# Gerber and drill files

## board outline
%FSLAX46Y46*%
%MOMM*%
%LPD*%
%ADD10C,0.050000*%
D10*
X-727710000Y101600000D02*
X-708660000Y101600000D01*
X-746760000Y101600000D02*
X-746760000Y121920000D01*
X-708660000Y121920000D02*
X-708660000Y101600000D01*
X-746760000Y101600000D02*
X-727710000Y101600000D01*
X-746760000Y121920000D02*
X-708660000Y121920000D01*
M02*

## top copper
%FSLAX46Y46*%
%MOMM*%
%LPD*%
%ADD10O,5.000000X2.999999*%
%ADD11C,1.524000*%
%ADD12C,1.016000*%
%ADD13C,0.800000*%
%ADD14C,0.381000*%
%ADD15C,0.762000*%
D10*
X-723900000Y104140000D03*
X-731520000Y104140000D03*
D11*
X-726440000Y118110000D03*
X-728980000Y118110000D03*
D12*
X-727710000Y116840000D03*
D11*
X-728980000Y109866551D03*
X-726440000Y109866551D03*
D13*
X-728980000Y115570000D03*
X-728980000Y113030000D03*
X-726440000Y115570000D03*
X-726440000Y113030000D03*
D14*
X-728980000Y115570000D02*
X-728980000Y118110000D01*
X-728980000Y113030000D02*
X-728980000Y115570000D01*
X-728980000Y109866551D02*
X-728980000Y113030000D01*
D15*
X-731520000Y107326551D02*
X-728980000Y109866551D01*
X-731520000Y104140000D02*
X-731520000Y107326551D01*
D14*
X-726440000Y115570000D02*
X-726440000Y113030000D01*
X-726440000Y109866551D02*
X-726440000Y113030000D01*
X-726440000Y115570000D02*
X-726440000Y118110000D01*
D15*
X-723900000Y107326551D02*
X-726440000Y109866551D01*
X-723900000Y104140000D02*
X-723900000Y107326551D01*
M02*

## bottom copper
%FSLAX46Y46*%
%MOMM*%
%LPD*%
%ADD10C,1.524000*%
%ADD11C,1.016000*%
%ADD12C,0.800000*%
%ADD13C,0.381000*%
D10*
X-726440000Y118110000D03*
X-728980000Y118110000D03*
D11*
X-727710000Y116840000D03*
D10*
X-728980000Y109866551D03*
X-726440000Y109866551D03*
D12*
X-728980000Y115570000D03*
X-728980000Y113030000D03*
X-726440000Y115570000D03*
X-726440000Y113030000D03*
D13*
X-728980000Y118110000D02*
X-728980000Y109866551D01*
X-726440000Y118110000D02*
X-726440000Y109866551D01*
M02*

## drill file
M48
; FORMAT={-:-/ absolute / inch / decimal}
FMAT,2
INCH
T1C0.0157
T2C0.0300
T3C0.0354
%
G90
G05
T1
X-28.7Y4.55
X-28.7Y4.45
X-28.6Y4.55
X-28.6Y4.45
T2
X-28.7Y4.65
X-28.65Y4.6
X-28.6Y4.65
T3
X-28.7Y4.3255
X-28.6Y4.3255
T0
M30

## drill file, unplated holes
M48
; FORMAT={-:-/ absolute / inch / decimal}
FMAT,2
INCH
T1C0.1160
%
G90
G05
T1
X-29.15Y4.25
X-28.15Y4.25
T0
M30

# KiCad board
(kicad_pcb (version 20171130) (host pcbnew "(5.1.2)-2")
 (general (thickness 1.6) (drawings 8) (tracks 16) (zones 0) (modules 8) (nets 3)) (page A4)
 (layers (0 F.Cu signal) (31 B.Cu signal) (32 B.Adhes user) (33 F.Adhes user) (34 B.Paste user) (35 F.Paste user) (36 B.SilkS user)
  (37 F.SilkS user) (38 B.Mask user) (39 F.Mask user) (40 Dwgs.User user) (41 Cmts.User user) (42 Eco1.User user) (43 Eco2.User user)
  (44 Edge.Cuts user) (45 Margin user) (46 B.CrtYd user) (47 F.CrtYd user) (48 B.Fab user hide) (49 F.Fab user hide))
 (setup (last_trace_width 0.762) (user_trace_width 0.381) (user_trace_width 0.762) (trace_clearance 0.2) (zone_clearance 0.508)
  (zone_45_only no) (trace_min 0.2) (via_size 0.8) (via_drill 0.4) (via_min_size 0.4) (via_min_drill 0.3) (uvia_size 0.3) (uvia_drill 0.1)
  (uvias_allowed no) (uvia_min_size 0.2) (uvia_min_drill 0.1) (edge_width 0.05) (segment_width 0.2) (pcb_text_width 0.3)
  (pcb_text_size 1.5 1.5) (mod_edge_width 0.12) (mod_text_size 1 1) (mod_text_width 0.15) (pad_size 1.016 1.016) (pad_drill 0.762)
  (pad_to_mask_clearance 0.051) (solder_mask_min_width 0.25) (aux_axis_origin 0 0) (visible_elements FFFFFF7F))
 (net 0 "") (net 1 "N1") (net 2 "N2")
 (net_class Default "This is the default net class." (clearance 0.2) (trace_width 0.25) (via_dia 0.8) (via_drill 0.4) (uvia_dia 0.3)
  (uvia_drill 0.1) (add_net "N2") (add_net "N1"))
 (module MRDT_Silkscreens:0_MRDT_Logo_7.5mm (layer F.Cu) (at -714.375 -116.84)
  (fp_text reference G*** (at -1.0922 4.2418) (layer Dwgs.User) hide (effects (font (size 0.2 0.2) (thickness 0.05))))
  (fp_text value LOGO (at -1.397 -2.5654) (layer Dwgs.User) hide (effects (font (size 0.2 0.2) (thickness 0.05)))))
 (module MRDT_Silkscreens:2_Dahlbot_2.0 (layer B.Cu) (at -740.41 -115.57 180)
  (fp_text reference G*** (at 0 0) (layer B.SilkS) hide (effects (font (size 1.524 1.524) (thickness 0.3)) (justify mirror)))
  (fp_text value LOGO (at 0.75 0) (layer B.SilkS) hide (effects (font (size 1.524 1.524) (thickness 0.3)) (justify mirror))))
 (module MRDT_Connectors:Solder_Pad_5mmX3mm (layer F.Cu) (at -723.9 -104.14 90)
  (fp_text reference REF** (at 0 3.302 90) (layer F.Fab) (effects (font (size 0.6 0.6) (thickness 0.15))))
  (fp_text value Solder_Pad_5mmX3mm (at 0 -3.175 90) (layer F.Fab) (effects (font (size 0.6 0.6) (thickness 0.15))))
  (pad 1 smd oval (at 0 0 90) (size 2.999999 5) (layers F.Cu F.Paste F.Mask) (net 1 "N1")))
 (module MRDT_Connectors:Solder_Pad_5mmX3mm (layer F.Cu) (at -731.52 -104.14 90)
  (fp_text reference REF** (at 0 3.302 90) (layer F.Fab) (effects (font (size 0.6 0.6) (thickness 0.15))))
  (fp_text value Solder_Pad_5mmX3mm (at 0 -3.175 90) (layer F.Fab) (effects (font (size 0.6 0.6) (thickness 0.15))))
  (pad 1 smd oval (at 0 0 90) (size 2.999999 5) (layers F.Cu F.Paste F.Mask) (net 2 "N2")))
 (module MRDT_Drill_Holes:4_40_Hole (layer F.Cu) (at -740.41 -107.95)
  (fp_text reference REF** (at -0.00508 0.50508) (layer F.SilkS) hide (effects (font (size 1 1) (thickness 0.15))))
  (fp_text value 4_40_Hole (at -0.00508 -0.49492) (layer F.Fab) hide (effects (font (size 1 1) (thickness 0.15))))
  (pad "" np_thru_hole circle (at 0 0) (size 2.9464 2.9464) (drill 2.9464) (layers *.Cu *.Mask)))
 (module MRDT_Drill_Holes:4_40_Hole (layer F.Cu) (at -715.01 -107.95)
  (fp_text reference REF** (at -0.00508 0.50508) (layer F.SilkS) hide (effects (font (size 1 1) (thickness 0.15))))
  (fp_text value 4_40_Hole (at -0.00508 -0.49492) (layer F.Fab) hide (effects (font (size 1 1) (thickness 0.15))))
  (pad "" np_thru_hole circle (at 0 0) (size 2.9464 2.9464) (drill 2.9464) (layers *.Cu *.Mask)))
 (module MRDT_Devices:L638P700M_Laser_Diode (layer B.Cu) (at -726.44 -118.11 180)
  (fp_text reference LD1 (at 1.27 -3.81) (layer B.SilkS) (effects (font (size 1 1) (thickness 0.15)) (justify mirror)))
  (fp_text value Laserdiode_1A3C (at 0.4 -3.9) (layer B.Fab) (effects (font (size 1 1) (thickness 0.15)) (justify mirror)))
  (pad 1 thru_hole circle (at 0 0 180) (size 1.524 1.524) (drill 0.762) (layers *.Cu *.Mask) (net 1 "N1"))
  (pad 3 thru_hole circle (at 2.54 0 180) (size 1.524 1.524) (drill 0.762) (layers *.Cu *.Mask) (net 2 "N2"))
  (pad 2 thru_hole circle (at 1.27 -1.27 180) (size 1.016 1.016) (drill 0.762) (layers *.Cu *.Mask)))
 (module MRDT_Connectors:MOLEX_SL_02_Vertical (layer F.Cu) (at -727.71 -109.866551)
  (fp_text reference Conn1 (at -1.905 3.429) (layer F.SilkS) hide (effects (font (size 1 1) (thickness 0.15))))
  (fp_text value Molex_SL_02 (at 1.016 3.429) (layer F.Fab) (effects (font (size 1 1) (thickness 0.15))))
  (pad 1 thru_hole circle (at -1.27 0) (size 1.524 1.524) (drill 0.9) (layers *.Cu *.Mask) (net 2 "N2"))
  (pad 2 thru_hole circle (at 1.27 0) (size 1.524 1.524) (drill 0.9) (layers *.Cu *.Mask) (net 1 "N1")))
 (gr_line (start -727.71 -101.6) (end -708.66 -101.6) (layer Edge.Cuts) (width 0.05))
 (gr_line (start -746.76 -101.6) (end -746.76 -121.92) (layer Edge.Cuts) (width 0.05))
 (gr_line (start -708.66 -121.92) (end -708.66 -101.6) (layer Edge.Cuts) (width 0.05))
 (gr_line (start -746.76 -101.6) (end -727.71 -101.6) (layer Edge.Cuts) (width 0.05))
 (gr_line (start -746.76 -121.92) (end -708.66 -121.92) (layer Edge.Cuts) (width 0.05))
 (via (at -728.98 -115.57) (size 0.8) (drill 0.4) (layers F.Cu B.Cu) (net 2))
 (via (at -728.98 -113.03) (size 0.8) (drill 0.4) (layers F.Cu B.Cu) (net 2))
 (segment (start -728.98 -118.11) (end -728.98 -109.866551) (width 0.381) (layer B.Cu) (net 2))
 (segment (start -728.98 -115.57) (end -728.98 -118.11) (width 0.381) (layer F.Cu) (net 2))
 (segment (start -728.98 -113.03) (end -728.98 -115.57) (width 0.381) (layer F.Cu) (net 2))
 (segment (start -728.98 -109.866551) (end -728.98 -113.03) (width 0.381) (layer F.Cu) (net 2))
 (segment (start -731.52 -107.326551) (end -728.98 -109.866551) (width 0.762) (layer F.Cu) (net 2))
 (segment (start -731.52 -104.14) (end -731.52 -107.326551) (width 0.762) (layer F.Cu) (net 2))
 (via (at -726.44 -115.57) (size 0.8) (drill 0.4) (layers F.Cu B.Cu) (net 1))
 (via (at -726.44 -113.03) (size 0.8) (drill 0.4) (layers F.Cu B.Cu) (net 1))
 (segment (start -726.44 -118.11) (end -726.44 -109.866551) (width 0.381) (layer B.Cu) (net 1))
 (segment (start -726.44 -115.57) (end -726.44 -113.03) (width 0.381) (layer F.Cu) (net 1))
 (segment (start -726.44 -109.866551) (end -726.44 -113.03) (width 0.381) (layer F.Cu) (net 1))
 (segment (start -726.44 -115.57) (end -726.44 -118.11) (width 0.381) (layer F.Cu) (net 1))
 (segment (start -723.9 -107.326551) (end -726.44 -109.866551) (width 0.762) (layer F.Cu) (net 1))
 (segment (start -723.9 -104.14) (end -723.9 -107.326551) (width 0.762) (layer F.Cu) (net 1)))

